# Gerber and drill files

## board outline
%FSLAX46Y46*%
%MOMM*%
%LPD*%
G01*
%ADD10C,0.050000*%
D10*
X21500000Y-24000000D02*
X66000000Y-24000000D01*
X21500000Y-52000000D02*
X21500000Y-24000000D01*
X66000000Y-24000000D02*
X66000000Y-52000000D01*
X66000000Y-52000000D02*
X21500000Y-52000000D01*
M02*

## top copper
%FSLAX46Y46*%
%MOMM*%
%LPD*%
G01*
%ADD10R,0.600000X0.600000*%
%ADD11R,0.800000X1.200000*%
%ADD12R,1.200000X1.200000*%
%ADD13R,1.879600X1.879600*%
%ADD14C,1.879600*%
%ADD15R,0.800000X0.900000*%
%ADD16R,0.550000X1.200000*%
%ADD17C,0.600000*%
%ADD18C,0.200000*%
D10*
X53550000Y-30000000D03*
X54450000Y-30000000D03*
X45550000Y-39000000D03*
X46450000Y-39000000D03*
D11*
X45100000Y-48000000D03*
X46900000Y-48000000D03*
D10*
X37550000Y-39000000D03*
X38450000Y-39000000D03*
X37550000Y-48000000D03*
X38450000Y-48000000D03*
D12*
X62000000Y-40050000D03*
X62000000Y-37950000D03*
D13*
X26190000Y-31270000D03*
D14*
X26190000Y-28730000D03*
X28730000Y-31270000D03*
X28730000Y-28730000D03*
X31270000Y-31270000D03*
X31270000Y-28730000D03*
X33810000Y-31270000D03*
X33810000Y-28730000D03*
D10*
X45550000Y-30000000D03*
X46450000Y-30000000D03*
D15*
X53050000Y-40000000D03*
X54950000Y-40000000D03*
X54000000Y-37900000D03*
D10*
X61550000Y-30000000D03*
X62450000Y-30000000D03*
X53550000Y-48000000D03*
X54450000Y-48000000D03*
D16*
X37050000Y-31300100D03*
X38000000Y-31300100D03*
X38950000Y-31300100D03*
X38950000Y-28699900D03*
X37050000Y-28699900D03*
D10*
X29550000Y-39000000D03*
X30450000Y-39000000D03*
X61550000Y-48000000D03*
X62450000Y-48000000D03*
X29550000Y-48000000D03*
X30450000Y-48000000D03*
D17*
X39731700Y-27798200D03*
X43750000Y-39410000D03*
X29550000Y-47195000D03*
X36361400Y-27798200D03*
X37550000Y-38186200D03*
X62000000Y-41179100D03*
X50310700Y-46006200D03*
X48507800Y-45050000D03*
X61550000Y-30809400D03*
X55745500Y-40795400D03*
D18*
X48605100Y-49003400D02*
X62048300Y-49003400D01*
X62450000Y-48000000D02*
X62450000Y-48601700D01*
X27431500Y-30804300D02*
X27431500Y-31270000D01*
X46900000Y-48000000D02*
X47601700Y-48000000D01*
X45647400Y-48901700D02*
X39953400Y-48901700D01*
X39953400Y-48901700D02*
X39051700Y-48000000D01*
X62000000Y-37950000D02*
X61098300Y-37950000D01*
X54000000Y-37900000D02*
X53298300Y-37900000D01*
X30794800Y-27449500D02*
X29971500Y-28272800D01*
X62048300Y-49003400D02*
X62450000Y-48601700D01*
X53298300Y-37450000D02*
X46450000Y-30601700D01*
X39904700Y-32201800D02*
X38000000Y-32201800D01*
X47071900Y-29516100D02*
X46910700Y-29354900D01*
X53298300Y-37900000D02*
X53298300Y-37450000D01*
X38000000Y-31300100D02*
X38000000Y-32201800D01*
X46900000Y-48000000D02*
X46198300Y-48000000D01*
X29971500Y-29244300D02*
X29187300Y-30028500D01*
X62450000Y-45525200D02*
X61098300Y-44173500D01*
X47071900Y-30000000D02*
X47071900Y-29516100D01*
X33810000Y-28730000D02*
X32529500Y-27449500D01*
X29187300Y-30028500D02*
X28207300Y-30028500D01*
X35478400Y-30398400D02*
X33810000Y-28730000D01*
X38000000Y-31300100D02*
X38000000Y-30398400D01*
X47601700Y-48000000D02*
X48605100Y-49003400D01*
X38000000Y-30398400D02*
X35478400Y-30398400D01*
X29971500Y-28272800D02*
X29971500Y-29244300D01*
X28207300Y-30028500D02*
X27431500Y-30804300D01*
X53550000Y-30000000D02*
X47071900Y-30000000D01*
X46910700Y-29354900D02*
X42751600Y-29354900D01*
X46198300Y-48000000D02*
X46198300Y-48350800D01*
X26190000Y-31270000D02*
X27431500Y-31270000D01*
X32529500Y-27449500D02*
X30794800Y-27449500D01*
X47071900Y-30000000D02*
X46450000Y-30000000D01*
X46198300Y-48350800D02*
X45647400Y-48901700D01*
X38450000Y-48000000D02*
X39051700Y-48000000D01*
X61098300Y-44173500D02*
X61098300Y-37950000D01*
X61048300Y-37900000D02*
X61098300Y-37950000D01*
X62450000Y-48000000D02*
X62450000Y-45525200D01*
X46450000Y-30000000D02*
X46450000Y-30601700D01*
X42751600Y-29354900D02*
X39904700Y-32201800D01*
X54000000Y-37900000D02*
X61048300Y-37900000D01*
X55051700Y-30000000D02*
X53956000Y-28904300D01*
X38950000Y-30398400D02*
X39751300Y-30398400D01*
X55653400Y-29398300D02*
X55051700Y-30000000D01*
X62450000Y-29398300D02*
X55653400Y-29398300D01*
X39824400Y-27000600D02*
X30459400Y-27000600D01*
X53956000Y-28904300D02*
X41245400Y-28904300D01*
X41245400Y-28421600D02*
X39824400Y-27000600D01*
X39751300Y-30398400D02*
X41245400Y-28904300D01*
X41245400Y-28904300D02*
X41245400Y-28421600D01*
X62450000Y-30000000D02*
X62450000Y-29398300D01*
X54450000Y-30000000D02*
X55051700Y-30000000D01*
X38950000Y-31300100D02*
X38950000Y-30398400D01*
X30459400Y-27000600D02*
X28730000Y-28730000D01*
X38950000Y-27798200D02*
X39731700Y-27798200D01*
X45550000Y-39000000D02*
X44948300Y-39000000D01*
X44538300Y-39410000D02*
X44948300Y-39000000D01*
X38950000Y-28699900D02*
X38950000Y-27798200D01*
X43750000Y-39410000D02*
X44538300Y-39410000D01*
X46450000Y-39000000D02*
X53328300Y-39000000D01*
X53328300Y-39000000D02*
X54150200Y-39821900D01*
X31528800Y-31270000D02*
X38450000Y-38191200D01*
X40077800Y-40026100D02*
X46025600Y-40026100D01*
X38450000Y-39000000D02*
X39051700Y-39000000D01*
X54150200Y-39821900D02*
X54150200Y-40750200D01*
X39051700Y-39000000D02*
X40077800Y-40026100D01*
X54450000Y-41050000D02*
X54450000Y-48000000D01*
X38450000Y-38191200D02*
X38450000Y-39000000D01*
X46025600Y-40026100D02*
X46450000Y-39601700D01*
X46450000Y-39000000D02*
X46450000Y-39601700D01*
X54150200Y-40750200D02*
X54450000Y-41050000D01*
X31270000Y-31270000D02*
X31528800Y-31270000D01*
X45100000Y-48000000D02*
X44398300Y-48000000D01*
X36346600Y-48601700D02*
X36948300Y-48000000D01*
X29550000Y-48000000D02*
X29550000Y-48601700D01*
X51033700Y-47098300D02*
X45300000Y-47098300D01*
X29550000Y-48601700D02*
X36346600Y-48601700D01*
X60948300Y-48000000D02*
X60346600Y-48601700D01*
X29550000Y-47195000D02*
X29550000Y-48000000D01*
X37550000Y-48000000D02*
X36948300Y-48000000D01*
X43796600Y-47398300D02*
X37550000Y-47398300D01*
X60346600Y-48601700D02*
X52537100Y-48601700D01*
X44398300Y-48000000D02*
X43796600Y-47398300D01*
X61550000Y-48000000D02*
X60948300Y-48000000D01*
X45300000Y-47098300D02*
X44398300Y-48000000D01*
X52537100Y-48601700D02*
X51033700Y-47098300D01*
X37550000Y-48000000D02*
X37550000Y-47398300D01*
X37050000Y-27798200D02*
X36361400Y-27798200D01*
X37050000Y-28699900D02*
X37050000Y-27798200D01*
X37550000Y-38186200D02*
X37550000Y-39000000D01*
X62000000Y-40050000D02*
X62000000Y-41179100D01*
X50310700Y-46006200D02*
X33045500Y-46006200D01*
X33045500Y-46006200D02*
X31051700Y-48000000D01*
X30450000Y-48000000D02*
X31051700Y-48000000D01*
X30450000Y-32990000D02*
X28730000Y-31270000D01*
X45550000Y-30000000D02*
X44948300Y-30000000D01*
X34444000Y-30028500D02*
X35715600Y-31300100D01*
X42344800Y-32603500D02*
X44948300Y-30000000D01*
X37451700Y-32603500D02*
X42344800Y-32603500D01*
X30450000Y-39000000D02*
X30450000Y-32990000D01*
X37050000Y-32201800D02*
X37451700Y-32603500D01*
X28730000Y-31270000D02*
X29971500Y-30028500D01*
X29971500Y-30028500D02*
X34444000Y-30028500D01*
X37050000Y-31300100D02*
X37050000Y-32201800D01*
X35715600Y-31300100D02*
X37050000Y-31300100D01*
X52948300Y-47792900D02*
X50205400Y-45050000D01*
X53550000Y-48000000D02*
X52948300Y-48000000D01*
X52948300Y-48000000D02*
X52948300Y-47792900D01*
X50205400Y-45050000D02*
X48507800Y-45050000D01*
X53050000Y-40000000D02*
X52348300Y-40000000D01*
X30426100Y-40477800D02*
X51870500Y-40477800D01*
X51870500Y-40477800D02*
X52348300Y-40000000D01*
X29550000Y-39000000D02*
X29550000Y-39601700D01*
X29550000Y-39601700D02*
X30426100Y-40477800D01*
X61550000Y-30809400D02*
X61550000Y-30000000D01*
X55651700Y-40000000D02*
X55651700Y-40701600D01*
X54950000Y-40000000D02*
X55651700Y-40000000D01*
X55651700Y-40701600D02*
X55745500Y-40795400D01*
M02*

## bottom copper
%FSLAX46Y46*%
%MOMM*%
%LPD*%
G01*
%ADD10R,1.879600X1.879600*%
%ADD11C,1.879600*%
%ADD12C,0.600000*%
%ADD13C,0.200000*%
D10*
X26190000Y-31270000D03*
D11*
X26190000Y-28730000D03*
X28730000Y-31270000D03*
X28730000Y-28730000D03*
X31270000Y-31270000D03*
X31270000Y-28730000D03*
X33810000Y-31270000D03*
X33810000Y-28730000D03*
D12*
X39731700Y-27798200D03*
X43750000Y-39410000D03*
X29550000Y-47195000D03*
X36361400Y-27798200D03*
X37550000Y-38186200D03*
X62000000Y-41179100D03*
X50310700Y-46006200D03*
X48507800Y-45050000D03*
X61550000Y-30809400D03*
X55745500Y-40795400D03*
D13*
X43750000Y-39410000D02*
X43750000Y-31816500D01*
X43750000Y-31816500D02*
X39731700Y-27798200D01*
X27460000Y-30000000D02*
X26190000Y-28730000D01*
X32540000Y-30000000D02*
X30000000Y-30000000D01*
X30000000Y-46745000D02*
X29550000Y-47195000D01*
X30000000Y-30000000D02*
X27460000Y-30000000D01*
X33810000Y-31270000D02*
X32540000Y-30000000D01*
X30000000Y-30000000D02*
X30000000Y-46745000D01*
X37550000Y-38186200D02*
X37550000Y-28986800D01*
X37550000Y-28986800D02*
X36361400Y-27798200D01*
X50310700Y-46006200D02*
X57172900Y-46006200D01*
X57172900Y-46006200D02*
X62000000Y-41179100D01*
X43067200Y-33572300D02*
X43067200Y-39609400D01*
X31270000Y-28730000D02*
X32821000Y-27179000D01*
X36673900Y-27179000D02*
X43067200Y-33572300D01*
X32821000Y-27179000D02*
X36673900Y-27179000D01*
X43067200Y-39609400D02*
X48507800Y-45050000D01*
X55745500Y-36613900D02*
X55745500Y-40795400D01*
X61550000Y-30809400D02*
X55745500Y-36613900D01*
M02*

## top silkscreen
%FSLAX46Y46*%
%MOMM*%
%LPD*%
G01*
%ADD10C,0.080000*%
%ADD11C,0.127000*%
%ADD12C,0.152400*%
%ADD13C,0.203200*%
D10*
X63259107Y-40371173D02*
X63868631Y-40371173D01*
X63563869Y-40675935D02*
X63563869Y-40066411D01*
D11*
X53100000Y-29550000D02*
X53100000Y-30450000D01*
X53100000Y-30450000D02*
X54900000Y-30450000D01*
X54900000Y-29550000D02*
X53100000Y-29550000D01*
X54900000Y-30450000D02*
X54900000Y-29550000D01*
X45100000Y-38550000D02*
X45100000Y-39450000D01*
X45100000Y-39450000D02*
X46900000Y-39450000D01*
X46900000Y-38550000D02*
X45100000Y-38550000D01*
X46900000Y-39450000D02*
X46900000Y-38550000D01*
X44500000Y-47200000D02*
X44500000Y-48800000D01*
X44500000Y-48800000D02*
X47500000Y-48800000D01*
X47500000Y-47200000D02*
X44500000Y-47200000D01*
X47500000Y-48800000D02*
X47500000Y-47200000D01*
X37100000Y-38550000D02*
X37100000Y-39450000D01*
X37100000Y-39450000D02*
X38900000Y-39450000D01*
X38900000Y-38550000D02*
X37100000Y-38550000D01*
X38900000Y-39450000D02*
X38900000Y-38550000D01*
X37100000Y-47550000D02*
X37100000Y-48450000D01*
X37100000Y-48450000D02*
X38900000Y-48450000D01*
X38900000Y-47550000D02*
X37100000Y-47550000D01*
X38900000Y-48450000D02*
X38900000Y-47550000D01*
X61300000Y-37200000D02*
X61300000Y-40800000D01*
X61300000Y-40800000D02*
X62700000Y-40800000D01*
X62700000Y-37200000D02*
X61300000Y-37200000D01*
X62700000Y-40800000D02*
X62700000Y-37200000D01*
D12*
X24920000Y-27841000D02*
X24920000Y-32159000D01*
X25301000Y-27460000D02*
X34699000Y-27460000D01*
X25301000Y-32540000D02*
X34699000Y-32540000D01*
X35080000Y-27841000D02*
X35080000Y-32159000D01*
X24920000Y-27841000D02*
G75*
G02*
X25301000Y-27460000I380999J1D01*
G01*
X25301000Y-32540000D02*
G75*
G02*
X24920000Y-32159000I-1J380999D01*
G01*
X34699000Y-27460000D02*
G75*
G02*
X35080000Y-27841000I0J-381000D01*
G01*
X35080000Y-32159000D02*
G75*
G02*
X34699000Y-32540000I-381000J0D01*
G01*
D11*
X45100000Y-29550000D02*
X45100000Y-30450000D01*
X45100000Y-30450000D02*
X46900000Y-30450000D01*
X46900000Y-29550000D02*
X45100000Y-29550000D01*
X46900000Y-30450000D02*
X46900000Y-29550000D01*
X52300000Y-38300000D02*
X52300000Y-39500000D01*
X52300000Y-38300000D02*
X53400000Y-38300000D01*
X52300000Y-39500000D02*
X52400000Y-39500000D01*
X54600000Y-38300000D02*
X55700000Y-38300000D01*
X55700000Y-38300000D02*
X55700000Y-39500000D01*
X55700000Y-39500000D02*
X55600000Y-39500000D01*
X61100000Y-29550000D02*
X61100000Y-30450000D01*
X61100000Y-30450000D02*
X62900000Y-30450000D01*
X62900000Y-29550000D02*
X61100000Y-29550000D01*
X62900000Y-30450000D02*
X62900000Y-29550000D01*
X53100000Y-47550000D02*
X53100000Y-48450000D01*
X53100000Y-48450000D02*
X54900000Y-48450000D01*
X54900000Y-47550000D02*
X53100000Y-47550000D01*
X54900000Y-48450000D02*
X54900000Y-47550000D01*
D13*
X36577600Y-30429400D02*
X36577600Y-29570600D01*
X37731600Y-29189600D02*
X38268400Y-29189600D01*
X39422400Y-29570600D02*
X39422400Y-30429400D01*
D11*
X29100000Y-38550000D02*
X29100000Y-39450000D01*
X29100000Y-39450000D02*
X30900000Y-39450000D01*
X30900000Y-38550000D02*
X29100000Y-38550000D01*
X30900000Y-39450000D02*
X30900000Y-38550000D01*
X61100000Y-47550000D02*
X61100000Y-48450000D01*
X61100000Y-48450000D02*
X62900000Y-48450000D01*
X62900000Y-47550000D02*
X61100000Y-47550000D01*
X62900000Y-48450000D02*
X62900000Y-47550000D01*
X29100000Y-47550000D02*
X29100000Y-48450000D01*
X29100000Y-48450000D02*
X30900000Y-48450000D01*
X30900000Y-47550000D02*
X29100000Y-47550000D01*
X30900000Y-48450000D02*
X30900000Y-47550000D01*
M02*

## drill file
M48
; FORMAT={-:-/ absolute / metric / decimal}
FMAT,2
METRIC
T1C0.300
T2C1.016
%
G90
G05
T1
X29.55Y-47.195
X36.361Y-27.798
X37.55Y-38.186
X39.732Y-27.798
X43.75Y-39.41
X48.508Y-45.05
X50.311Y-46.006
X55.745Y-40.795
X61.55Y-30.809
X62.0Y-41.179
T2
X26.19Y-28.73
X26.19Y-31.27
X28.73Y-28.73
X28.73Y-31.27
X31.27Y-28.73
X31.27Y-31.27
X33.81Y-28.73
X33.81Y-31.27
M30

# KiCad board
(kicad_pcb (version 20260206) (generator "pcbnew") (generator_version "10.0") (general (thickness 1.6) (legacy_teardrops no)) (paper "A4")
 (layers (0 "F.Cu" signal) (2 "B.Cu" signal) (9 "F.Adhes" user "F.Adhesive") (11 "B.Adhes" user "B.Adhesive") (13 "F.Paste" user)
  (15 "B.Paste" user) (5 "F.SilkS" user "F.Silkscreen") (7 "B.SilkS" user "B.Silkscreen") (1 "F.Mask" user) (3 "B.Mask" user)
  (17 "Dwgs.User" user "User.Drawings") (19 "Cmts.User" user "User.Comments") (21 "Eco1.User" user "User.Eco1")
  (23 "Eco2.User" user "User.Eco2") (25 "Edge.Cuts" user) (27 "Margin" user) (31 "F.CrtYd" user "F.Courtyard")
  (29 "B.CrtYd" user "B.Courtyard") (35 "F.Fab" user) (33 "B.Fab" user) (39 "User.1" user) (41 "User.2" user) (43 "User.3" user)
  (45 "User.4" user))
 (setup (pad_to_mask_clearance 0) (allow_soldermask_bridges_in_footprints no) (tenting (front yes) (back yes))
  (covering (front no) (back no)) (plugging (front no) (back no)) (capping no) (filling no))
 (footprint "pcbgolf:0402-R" (layer "F.Cu") (at 54 30)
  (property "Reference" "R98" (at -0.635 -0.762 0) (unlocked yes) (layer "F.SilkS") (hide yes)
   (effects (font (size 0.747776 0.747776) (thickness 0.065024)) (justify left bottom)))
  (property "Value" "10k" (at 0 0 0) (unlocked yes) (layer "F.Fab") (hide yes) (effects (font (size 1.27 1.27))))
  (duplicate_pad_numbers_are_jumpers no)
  (fp_line (start -0.9 -0.45) (end -0.9 0.45) (stroke (width 0.127) (type solid)) (layer "F.SilkS"))
  (fp_line (start -0.9 0.45) (end 0.9 0.45) (stroke (width 0.127) (type solid)) (layer "F.SilkS"))
  (fp_line (start 0.9 -0.45) (end -0.9 -0.45) (stroke (width 0.127) (type solid)) (layer "F.SilkS"))
  (fp_line (start 0.9 0.45) (end 0.9 -0.45) (stroke (width 0.127) (type solid)) (layer "F.SilkS"))
  (pad "1" smd rect (at -0.45 0) (size 0.6 0.6) (layers "F.Cu" "F.Mask" "F.Paste") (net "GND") (solder_mask_margin 0.0508)
   (solder_paste_margin 0) (thermal_bridge_angle 0))
  (pad "2" smd rect (at 0.45 0) (size 0.6 0.6) (layers "F.Cu" "F.Mask" "F.Paste") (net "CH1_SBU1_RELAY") (solder_mask_margin 0.0508)
   (solder_paste_margin 0) (thermal_bridge_angle 0)))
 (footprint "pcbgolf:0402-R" (layer "F.Cu") (at 46 39)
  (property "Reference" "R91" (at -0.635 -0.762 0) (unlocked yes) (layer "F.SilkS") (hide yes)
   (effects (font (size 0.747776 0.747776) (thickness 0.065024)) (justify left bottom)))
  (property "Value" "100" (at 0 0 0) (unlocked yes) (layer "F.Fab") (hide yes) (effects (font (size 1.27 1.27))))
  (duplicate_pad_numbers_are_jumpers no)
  (fp_line (start -0.9 -0.45) (end -0.9 0.45) (stroke (width 0.127) (type solid)) (layer "F.SilkS"))
  (fp_line (start -0.9 0.45) (end 0.9 0.45) (stroke (width 0.127) (type solid)) (layer "F.SilkS"))
  (fp_line (start 0.9 -0.45) (end -0.9 -0.45) (stroke (width 0.127) (type solid)) (layer "F.SilkS"))
  (fp_line (start 0.9 0.45) (end 0.9 -0.45) (stroke (width 0.127) (type solid)) (layer "F.SilkS"))
  (pad "1" smd rect (at -0.45 0) (size 0.6 0.6) (layers "F.Cu" "F.Mask" "F.Paste") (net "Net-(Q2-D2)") (solder_mask_margin 0.0508)
   (solder_paste_margin 0) (thermal_bridge_angle 0))
  (pad "2" smd rect (at 0.45 0) (size 0.6 0.6) (layers "F.Cu" "F.Mask" "F.Paste") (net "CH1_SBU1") (solder_mask_margin 0.0508)
   (solder_paste_margin 0) (thermal_bridge_angle 0)))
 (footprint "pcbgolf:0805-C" (layer "F.Cu") (at 46 48)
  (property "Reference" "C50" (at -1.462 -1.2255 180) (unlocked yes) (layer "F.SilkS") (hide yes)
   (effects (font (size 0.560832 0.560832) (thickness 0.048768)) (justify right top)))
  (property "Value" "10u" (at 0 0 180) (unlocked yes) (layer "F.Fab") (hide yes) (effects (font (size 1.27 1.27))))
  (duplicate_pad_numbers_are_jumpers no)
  (fp_line (start -1.5 -0.8) (end -1.5 0.8) (stroke (width 0.127) (type solid)) (layer "F.SilkS"))
  (fp_line (start -1.5 0.8) (end 1.5 0.8) (stroke (width 0.127) (type solid)) (layer "F.SilkS"))
  (fp_line (start 1.5 -0.8) (end -1.5 -0.8) (stroke (width 0.127) (type solid)) (layer "F.SilkS"))
  (fp_line (start 1.5 0.8) (end 1.5 -0.8) (stroke (width 0.127) (type solid)) (layer "F.SilkS"))
  (pad "1" smd rect (at -0.9 0) (size 0.8 1.2) (layers "F.Cu" "F.Mask" "F.Paste") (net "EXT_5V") (solder_mask_margin 0.0508)
   (solder_paste_margin 0) (thermal_bridge_angle 0))
  (pad "2" smd rect (at 0.9 0) (size 0.8 1.2) (layers "F.Cu" "F.Mask" "F.Paste") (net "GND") (solder_mask_margin 0.0508)
   (solder_paste_margin 0) (thermal_bridge_angle 0)))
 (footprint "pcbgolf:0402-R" (layer "F.Cu") (at 38 39)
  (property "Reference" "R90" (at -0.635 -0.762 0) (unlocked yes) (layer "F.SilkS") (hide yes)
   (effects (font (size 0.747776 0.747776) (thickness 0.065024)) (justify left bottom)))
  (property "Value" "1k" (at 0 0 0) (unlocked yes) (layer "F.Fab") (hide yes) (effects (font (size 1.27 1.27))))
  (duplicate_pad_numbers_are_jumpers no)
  (fp_line (start -0.9 -0.45) (end -0.9 0.45) (stroke (width 0.127) (type solid)) (layer "F.SilkS"))
  (fp_line (start -0.9 0.45) (end 0.9 0.45) (stroke (width 0.127) (type solid)) (layer "F.SilkS"))
  (fp_line (start 0.9 -0.45) (end -0.9 -0.45) (stroke (width 0.127) (type solid)) (layer "F.SilkS"))
  (fp_line (start 0.9 0.45) (end 0.9 -0.45) (stroke (width 0.127) (type solid)) (layer "F.SilkS"))
  (pad "1" smd rect (at -0.45 0) (size 0.6 0.6) (layers "F.Cu" "F.Mask" "F.Paste") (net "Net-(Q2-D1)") (solder_mask_margin 0.0508)
   (solder_paste_margin 0) (thermal_bridge_angle 0))
  (pad "2" smd rect (at 0.45 0) (size 0.6 0.6) (layers "F.Cu" "F.Mask" "F.Paste") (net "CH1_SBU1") (solder_mask_margin 0.0508)
   (solder_paste_margin 0) (thermal_bridge_angle 0)))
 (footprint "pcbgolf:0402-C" (layer "F.Cu") (at 38 48)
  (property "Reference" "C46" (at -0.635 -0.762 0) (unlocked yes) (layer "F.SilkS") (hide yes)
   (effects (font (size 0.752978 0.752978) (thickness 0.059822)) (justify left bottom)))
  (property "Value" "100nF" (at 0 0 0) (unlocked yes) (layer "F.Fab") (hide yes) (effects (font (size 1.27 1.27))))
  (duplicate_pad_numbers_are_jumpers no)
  (fp_line (start -0.9 -0.45) (end -0.9 0.45) (stroke (width 0.127) (type solid)) (layer "F.SilkS"))
  (fp_line (start -0.9 0.45) (end 0.9 0.45) (stroke (width 0.127) (type solid)) (layer "F.SilkS"))
  (fp_line (start 0.9 -0.45) (end -0.9 -0.45) (stroke (width 0.127) (type solid)) (layer "F.SilkS"))
  (fp_line (start 0.9 0.45) (end 0.9 -0.45) (stroke (width 0.127) (type solid)) (layer "F.SilkS"))
  (pad "1" smd rect (at -0.45 0) (size 0.6 0.6) (layers "F.Cu" "F.Mask" "F.Paste") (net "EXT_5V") (solder_mask_margin 0.0508)
   (solder_paste_margin 0) (thermal_bridge_angle 0))
  (pad "2" smd rect (at 0.45 0) (size 0.6 0.6) (layers "F.Cu" "F.Mask" "F.Paste") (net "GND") (solder_mask_margin 0.0508)
   (solder_paste_margin 0) (thermal_bridge_angle 0)))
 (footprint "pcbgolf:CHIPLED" (layer "F.Cu") (at 62 39)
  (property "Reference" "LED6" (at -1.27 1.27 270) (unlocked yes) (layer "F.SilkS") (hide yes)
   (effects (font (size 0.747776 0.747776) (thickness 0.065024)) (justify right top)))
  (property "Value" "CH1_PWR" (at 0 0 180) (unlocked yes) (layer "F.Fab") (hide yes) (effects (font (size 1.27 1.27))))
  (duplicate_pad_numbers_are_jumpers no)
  (fp_line (start -0.7 -1.8) (end -0.7 1.8) (stroke (width 0.127) (type solid)) (layer "F.SilkS"))
  (fp_line (start -0.7 1.8) (end 0.7 1.8) (stroke (width 0.127) (type solid)) (layer "F.SilkS"))
  (fp_line (start 0.7 -1.8) (end -0.7 -1.8) (stroke (width 0.127) (type solid)) (layer "F.SilkS"))
  (fp_line (start 0.7 1.8) (end 0.7 -1.8) (stroke (width 0.127) (type solid)) (layer "F.SilkS"))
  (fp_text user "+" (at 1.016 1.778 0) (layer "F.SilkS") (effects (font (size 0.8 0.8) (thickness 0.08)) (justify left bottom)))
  (pad "A" smd rect (at 0 1.05) (size 1.2 1.2) (layers "F.Cu" "F.Mask" "F.Paste") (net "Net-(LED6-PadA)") (solder_mask_margin 0.0508)
   (solder_paste_margin 0) (thermal_bridge_angle 0))
  (pad "C" smd rect (at 0 -1.05) (size 1.2 1.2) (layers "F.Cu" "F.Mask" "F.Paste") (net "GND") (solder_mask_margin 0.0508)
   (solder_paste_margin 0) (thermal_bridge_angle 0)))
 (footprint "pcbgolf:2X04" (layer "F.Cu") (at 30 30)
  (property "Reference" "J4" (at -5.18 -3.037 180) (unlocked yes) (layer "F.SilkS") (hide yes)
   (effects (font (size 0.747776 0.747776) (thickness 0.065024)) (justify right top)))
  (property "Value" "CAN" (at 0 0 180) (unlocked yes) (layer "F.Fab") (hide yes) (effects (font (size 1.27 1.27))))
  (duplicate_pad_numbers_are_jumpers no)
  (fp_line (start -5.08 -2.159) (end -5.08 2.159) (stroke (width 0.1524) (type solid)) (layer "F.SilkS"))
  (fp_line (start -4.699 -2.54) (end 4.699 -2.54) (stroke (width 0.1524) (type solid)) (layer "F.SilkS"))
  (fp_line (start -4.699 2.54) (end 4.699 2.54) (stroke (width 0.1524) (type solid)) (layer "F.SilkS"))
  (fp_line (start 5.08 -2.159) (end 5.08 2.159) (stroke (width 0.1524) (type solid)) (layer "F.SilkS"))
  (fp_arc (start -5.08 -2.159) (mid -4.968408 -2.428408) (end -4.699 -2.54) (stroke (width 0.1524) (type solid)) (layer "F.SilkS"))
  (fp_arc (start -4.699 2.54) (mid -4.968408 2.428408) (end -5.08 2.159) (stroke (width 0.1524) (type solid)) (layer "F.SilkS"))
  (fp_arc (start 4.699 -2.54) (mid 4.968408 -2.428408) (end 5.08 -2.159) (stroke (width 0.1524) (type solid)) (layer "F.SilkS"))
  (fp_arc (start 5.08 2.159) (mid 4.968408 2.428408) (end 4.699 2.54) (stroke (width 0.1524) (type solid)) (layer "F.SilkS"))
  (pad "1" thru_hole rect (at -3.81 1.27 90) (size 1.8796 1.8796) (drill 1.016) (layers "*.Cu" "*.Mask") (remove_unused_layers no)
   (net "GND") (solder_mask_margin 0.0508) (thermal_bridge_angle 0))
  (pad "2" thru_hole circle (at -3.81 -1.27 90) (size 1.8796 1.8796) (drill 1.016) (layers "*.Cu" "*.Mask") (remove_unused_layers no)
   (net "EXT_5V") (solder_mask_margin 0.0508) (thermal_bridge_angle 0))
  (pad "3" thru_hole circle (at -1.27 1.27 90) (size 1.8796 1.8796) (drill 1.016) (layers "*.Cu" "*.Mask") (remove_unused_layers no)
   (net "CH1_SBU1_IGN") (solder_mask_margin 0.0508) (thermal_bridge_angle 0))
  (pad "4" thru_hole circle (at -1.27 -1.27 90) (size 1.8796 1.8796) (drill 1.016) (layers "*.Cu" "*.Mask") (remove_unused_layers no)
   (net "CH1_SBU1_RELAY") (solder_mask_margin 0.0508) (thermal_bridge_angle 0))
  (pad "5" thru_hole circle (at 1.27 1.27 90) (size 1.8796 1.8796) (drill 1.016) (layers "*.Cu" "*.Mask") (remove_unused_layers no)
   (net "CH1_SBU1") (solder_mask_margin 0.0508) (thermal_bridge_angle 0))
  (pad "6" thru_hole circle (at 1.27 -1.27 90) (size 1.8796 1.8796) (drill 1.016) (layers "*.Cu" "*.Mask") (remove_unused_layers no)
   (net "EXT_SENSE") (solder_mask_margin 0.0508) (thermal_bridge_angle 0))
  (pad "7" thru_hole circle (at 3.81 1.27 90) (size 1.8796 1.8796) (drill 1.016) (layers "*.Cu" "*.Mask") (remove_unused_layers no)
   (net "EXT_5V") (solder_mask_margin 0.0508) (thermal_bridge_angle 0))
  (pad "8" thru_hole circle (at 3.81 -1.27 90) (size 1.8796 1.8796) (drill 1.016) (layers "*.Cu" "*.Mask") (remove_unused_layers no)
   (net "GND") (solder_mask_margin 0.0508) (thermal_bridge_angle 0)))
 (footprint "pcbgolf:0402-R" (layer "F.Cu") (at 46 30)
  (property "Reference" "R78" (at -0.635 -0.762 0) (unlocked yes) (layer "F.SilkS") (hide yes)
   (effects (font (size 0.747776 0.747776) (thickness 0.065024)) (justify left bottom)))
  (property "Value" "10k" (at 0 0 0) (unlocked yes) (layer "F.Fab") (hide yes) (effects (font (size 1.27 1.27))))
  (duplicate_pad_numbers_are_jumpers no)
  (fp_line (start -0.9 -0.45) (end -0.9 0.45) (stroke (width 0.127) (type solid)) (layer "F.SilkS"))
  (fp_line (start -0.9 0.45) (end 0.9 0.45) (stroke (width 0.127) (type solid)) (layer "F.SilkS"))
  (fp_line (start 0.9 -0.45) (end -0.9 -0.45) (stroke (width 0.127) (type solid)) (layer "F.SilkS"))
  (fp_line (start 0.9 0.45) (end 0.9 -0.45) (stroke (width 0.127) (type solid)) (layer "F.SilkS"))
  (pad "1" smd rect (at -0.45 0) (size 0.6 0.6) (layers "F.Cu" "F.Mask" "F.Paste") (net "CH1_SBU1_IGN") (solder_mask_margin 0.0508)
   (solder_paste_margin 0) (thermal_bridge_angle 0))
  (pad "2" smd rect (at 0.45 0) (size 0.6 0.6) (layers "F.Cu" "F.Mask" "F.Paste") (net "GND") (solder_mask_margin 0.0508)
   (solder_paste_margin 0) (thermal_bridge_angle 0)))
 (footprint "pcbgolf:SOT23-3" (layer "F.Cu") (at 54 39)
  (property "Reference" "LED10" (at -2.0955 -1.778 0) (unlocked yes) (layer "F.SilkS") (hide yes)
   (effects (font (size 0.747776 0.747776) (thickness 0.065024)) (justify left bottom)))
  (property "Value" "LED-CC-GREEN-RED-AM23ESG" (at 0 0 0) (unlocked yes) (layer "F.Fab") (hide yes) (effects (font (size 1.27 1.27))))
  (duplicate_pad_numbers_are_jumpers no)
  (fp_line (start -1.7 -0.7) (end -1.7 0.5) (stroke (width 0.127) (type solid)) (layer "F.SilkS"))
  (fp_line (start -1.7 -0.7) (end -0.6 -0.7) (stroke (width 0.127) (type solid)) (layer "F.SilkS"))
  (fp_line (start -1.7 0.5) (end -1.6 0.5) (stroke (width 0.127) (type solid)) (layer "F.SilkS"))
  (fp_line (start 0.6 -0.7) (end 1.7 -0.7) (stroke (width 0.127) (type solid)) (layer "F.SilkS"))
  (fp_line (start 1.7 -0.7) (end 1.7 0.5) (stroke (width 0.127) (type solid)) (layer "F.SilkS"))
  (fp_line (start 1.7 0.5) (end 1.6 0.5) (stroke (width 0.127) (type solid)) (layer "F.SilkS"))
  (pad "1" smd rect (at -0.95 1) (size 0.8 0.9) (layers "F.Cu" "F.Mask" "F.Paste") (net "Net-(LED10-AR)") (solder_mask_margin 0.0508)
   (solder_paste_margin 0) (thermal_bridge_angle 0))
  (pad "2" smd rect (at 0.95 1) (size 0.8 0.9) (layers "F.Cu" "F.Mask" "F.Paste") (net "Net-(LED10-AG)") (solder_mask_margin 0.0508)
   (solder_paste_margin 0) (thermal_bridge_angle 0))
  (pad "3" smd rect (at 0 -1.1) (size 0.8 0.9) (layers "F.Cu" "F.Mask" "F.Paste") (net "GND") (solder_mask_margin 0.0508)
   (solder_paste_margin 0) (thermal_bridge_angle 0)))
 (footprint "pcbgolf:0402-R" (layer "F.Cu") (at 62 30)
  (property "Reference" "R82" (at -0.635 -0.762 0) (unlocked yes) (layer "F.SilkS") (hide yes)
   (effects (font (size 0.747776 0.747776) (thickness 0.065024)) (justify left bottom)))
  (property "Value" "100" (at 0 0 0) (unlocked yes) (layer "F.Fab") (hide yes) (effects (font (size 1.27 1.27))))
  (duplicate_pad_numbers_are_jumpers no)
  (fp_line (start -0.9 -0.45) (end -0.9 0.45) (stroke (width 0.127) (type solid)) (layer "F.SilkS"))
  (fp_line (start -0.9 0.45) (end 0.9 0.45) (stroke (width 0.127) (type solid)) (layer "F.SilkS"))
  (fp_line (start 0.9 -0.45) (end -0.9 -0.45) (stroke (width 0.127) (type solid)) (layer "F.SilkS"))
  (fp_line (start 0.9 0.45) (end 0.9 -0.45) (stroke (width 0.127) (type solid)) (layer "F.SilkS"))
  (pad "1" smd rect (at -0.45 0) (size 0.6 0.6) (layers "F.Cu" "F.Mask" "F.Paste") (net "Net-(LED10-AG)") (solder_mask_margin 0.0508)
   (solder_paste_margin 0) (thermal_bridge_angle 0))
  (pad "2" smd rect (at 0.45 0) (size 0.6 0.6) (layers "F.Cu" "F.Mask" "F.Paste") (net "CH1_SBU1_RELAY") (solder_mask_margin 0.0508)
   (solder_paste_margin 0) (thermal_bridge_angle 0)))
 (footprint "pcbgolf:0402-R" (layer "F.Cu") (at 54 48)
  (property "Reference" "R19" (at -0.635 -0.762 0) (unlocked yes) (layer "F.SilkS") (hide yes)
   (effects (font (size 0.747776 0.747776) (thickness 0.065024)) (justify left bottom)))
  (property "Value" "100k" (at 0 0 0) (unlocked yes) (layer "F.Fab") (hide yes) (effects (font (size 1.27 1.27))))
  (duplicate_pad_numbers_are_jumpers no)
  (fp_line (start -0.9 -0.45) (end -0.9 0.45) (stroke (width 0.127) (type solid)) (layer "F.SilkS"))
  (fp_line (start -0.9 0.45) (end 0.9 0.45) (stroke (width 0.127) (type solid)) (layer "F.SilkS"))
  (fp_line (start 0.9 -0.45) (end -0.9 -0.45) (stroke (width 0.127) (type solid)) (layer "F.SilkS"))
  (fp_line (start 0.9 0.45) (end 0.9 -0.45) (stroke (width 0.127) (type solid)) (layer "F.SilkS"))
  (pad "1" smd rect (at -0.45 0) (size 0.6 0.6) (layers "F.Cu" "F.Mask" "F.Paste") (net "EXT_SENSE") (solder_mask_margin 0.0508)
   (solder_paste_margin 0) (thermal_bridge_angle 0))
  (pad "2" smd rect (at 0.45 0) (size 0.6 0.6) (layers "F.Cu" "F.Mask" "F.Paste") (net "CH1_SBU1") (solder_mask_margin 0.0508)
   (solder_paste_margin 0) (thermal_bridge_angle 0)))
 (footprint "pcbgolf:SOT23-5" (layer "F.Cu") (at 38 30)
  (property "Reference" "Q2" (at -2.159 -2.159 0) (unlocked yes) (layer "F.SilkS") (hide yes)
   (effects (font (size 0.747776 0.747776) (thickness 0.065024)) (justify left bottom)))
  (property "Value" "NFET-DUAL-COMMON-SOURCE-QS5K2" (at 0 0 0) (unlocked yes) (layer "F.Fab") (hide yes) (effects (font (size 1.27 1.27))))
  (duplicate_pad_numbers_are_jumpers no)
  (fp_line (start -1.4224 0.4294) (end -1.4224 -0.4294) (stroke (width 0.2032) (type solid)) (layer "F.SilkS"))
  (fp_line (start -0.2684 -0.8104) (end 0.2684 -0.8104) (stroke (width 0.2032) (type solid)) (layer "F.SilkS"))
  (fp_line (start 1.4224 -0.4294) (end 1.4224 0.4294) (stroke (width 0.2032) (type solid)) (layer "F.SilkS"))
  (pad "1" smd rect (at -0.95 1.3001) (size 0.55 1.2) (layers "F.Cu" "F.Mask" "F.Paste") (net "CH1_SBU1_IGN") (solder_mask_margin 0.0508)
   (solder_paste_margin 0) (thermal_bridge_angle 0))
  (pad "2" smd rect (at 0 1.3001) (size 0.55 1.2) (layers "F.Cu" "F.Mask" "F.Paste") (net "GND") (solder_mask_margin 0.0508)
   (solder_paste_margin 0) (thermal_bridge_angle 0))
  (pad "3" smd rect (at 0.95 1.3001) (size 0.55 1.2) (layers "F.Cu" "F.Mask" "F.Paste") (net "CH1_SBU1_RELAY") (solder_mask_margin 0.0508)
   (solder_paste_margin 0) (thermal_bridge_angle 0))
  (pad "4" smd rect (at 0.95 -1.3001) (size 0.55 1.2) (layers "F.Cu" "F.Mask" "F.Paste") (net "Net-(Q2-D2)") (solder_mask_margin 0.0508)
   (solder_paste_margin 0) (thermal_bridge_angle 0))
  (pad "5" smd rect (at -0.95 -1.3001) (size 0.55 1.2) (layers "F.Cu" "F.Mask" "F.Paste") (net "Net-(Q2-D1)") (solder_mask_margin 0.0508)
   (solder_paste_margin 0) (thermal_bridge_angle 0)))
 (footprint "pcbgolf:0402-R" (layer "F.Cu") (at 30 39)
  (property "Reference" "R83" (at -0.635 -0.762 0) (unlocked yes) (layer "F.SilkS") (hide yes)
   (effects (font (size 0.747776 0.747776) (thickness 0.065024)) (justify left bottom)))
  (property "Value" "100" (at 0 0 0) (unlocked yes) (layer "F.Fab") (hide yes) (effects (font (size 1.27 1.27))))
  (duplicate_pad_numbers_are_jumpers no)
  (fp_line (start -0.9 -0.45) (end -0.9 0.45) (stroke (width 0.127) (type solid)) (layer "F.SilkS"))
  (fp_line (start -0.9 0.45) (end 0.9 0.45) (stroke (width 0.127) (type solid)) (layer "F.SilkS"))
  (fp_line (start 0.9 -0.45) (end -0.9 -0.45) (stroke (width 0.127) (type solid)) (layer "F.SilkS"))
  (fp_line (start 0.9 0.45) (end 0.9 -0.45) (stroke (width 0.127) (type solid)) (layer "F.SilkS"))
  (pad "1" smd rect (at -0.45 0) (size 0.6 0.6) (layers "F.Cu" "F.Mask" "F.Paste") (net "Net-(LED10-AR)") (solder_mask_margin 0.0508)
   (solder_paste_margin 0) (thermal_bridge_angle 0))
  (pad "2" smd rect (at 0.45 0) (size 0.6 0.6) (layers "F.Cu" "F.Mask" "F.Paste") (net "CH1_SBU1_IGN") (solder_mask_margin 0.0508)
   (solder_paste_margin 0) (thermal_bridge_angle 0)))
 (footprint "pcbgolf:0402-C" (layer "F.Cu") (at 62 48)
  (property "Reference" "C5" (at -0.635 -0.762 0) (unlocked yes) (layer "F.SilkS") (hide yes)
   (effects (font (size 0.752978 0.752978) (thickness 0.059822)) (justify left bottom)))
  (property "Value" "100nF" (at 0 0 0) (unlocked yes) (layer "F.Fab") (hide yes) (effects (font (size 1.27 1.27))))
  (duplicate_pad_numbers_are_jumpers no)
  (fp_line (start -0.9 -0.45) (end -0.9 0.45) (stroke (width 0.127) (type solid)) (layer "F.SilkS"))
  (fp_line (start -0.9 0.45) (end 0.9 0.45) (stroke (width 0.127) (type solid)) (layer "F.SilkS"))
  (fp_line (start 0.9 -0.45) (end -0.9 -0.45) (stroke (width 0.127) (type solid)) (layer "F.SilkS"))
  (fp_line (start 0.9 0.45) (end 0.9 -0.45) (stroke (width 0.127) (type solid)) (layer "F.SilkS"))
  (pad "1" smd rect (at -0.45 0) (size 0.6 0.6) (layers "F.Cu" "F.Mask" "F.Paste") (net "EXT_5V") (solder_mask_margin 0.0508)
   (solder_paste_margin 0) (thermal_bridge_angle 0))
  (pad "2" smd rect (at 0.45 0) (size 0.6 0.6) (layers "F.Cu" "F.Mask" "F.Paste") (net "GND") (solder_mask_margin 0.0508)
   (solder_paste_margin 0) (thermal_bridge_angle 0)))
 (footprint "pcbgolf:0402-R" (layer "F.Cu") (at 30 48)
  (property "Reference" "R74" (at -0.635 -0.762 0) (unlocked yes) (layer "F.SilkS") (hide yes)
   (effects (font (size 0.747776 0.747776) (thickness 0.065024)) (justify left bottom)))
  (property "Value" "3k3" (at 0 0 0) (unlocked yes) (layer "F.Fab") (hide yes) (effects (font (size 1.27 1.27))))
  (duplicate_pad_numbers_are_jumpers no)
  (fp_line (start -0.9 -0.45) (end -0.9 0.45) (stroke (width 0.127) (type solid)) (layer "F.SilkS"))
  (fp_line (start -0.9 0.45) (end 0.9 0.45) (stroke (width 0.127) (type solid)) (layer "F.SilkS"))
  (fp_line (start 0.9 -0.45) (end -0.9 -0.45) (stroke (width 0.127) (type solid)) (layer "F.SilkS"))
  (fp_line (start 0.9 0.45) (end 0.9 -0.45) (stroke (width 0.127) (type solid)) (layer "F.SilkS"))
  (pad "1" smd rect (at -0.45 0) (size 0.6 0.6) (layers "F.Cu" "F.Mask" "F.Paste") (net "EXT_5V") (solder_mask_margin 0.0508)
   (solder_paste_margin 0) (thermal_bridge_angle 0))
  (pad "2" smd rect (at 0.45 0) (size 0.6 0.6) (layers "F.Cu" "F.Mask" "F.Paste") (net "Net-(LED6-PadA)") (solder_mask_margin 0.0508)
   (solder_paste_margin 0) (thermal_bridge_angle 0)))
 (gr_line (start 21.5 24) (end 66 24) (stroke (width 0.05) (type default)) (layer "Edge.Cuts"))
 (gr_line (start 21.5 52) (end 21.5 24) (stroke (width 0.05) (type default)) (layer "Edge.Cuts"))
 (gr_line (start 66 24) (end 66 52) (stroke (width 0.05) (type default)) (layer "Edge.Cuts"))
 (gr_line (start 66 52) (end 21.5 52) (stroke (width 0.05) (type default)) (layer "Edge.Cuts"))
 (segment (start 48.6051 49.0034) (end 62.0483 49.0034) (width 0.2) (layer "F.Cu") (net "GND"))
 (segment (start 62.45 48) (end 62.45 48.6017) (width 0.2) (layer "F.Cu") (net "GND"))
 (segment (start 27.4315 30.8043) (end 27.4315 31.27) (width 0.2) (layer "F.Cu") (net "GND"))
 (segment (start 46.9 48) (end 47.6017 48) (width 0.2) (layer "F.Cu") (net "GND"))
 (segment (start 45.6474 48.9017) (end 39.9534 48.9017) (width 0.2) (layer "F.Cu") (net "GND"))
 (segment (start 39.9534 48.9017) (end 39.0517 48) (width 0.2) (layer "F.Cu") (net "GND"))
 (segment (start 62 37.95) (end 61.0983 37.95) (width 0.2) (layer "F.Cu") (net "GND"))
 (segment (start 54 37.9) (end 53.2983 37.9) (width 0.2) (layer "F.Cu") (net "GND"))
 (segment (start 30.7948 27.4495) (end 29.9715 28.2728) (width 0.2) (layer "F.Cu") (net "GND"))
 (segment (start 62.0483 49.0034) (end 62.45 48.6017) (width 0.2) (layer "F.Cu") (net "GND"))
 (segment (start 53.2983 37.45) (end 46.45 30.6017) (width 0.2) (layer "F.Cu") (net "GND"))
 (segment (start 39.9047 32.2018) (end 38 32.2018) (width 0.2) (layer "F.Cu") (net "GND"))
 (segment (start 47.0719 29.5161) (end 46.9107 29.3549) (width 0.2) (layer "F.Cu") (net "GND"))
 (segment (start 53.2983 37.9) (end 53.2983 37.45) (width 0.2) (layer "F.Cu") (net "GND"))
 (segment (start 38 31.3001) (end 38 32.2018) (width 0.2) (layer "F.Cu") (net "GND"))
 (segment (start 46.9 48) (end 46.1983 48) (width 0.2) (layer "F.Cu") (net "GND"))
 (segment (start 29.9715 29.2443) (end 29.1873 30.0285) (width 0.2) (layer "F.Cu") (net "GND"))
 (segment (start 62.45 45.5252) (end 61.0983 44.1735) (width 0.2) (layer "F.Cu") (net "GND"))
 (segment (start 47.0719 30) (end 47.0719 29.5161) (width 0.2) (layer "F.Cu") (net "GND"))
 (segment (start 33.81 28.73) (end 32.5295 27.4495) (width 0.2) (layer "F.Cu") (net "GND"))
 (segment (start 29.1873 30.0285) (end 28.2073 30.0285) (width 0.2) (layer "F.Cu") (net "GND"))
 (segment (start 35.4784 30.3984) (end 33.81 28.73) (width 0.2) (layer "F.Cu") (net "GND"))
 (segment (start 38 31.3001) (end 38 30.3984) (width 0.2) (layer "F.Cu") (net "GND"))
 (segment (start 47.6017 48) (end 48.6051 49.0034) (width 0.2) (layer "F.Cu") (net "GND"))
 (segment (start 38 30.3984) (end 35.4784 30.3984) (width 0.2) (layer "F.Cu") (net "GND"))
 (segment (start 29.9715 28.2728) (end 29.9715 29.2443) (width 0.2) (layer "F.Cu") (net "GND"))
 (segment (start 28.2073 30.0285) (end 27.4315 30.8043) (width 0.2) (layer "F.Cu") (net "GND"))
 (segment (start 53.55 30) (end 47.0719 30) (width 0.2) (layer "F.Cu") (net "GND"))
 (segment (start 46.9107 29.3549) (end 42.7516 29.3549) (width 0.2) (layer "F.Cu") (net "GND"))
 (segment (start 46.1983 48) (end 46.1983 48.3508) (width 0.2) (layer "F.Cu") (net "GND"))
 (segment (start 26.19 31.27) (end 27.4315 31.27) (width 0.2) (layer "F.Cu") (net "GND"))
 (segment (start 32.5295 27.4495) (end 30.7948 27.4495) (width 0.2) (layer "F.Cu") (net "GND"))
 (segment (start 47.0719 30) (end 46.45 30) (width 0.2) (layer "F.Cu") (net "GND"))
 (segment (start 46.1983 48.3508) (end 45.6474 48.9017) (width 0.2) (layer "F.Cu") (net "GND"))
 (segment (start 38.45 48) (end 39.0517 48) (width 0.2) (layer "F.Cu") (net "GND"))
 (segment (start 61.0983 44.1735) (end 61.0983 37.95) (width 0.2) (layer "F.Cu") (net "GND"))
 (segment (start 61.0483 37.9) (end 61.0983 37.95) (width 0.2) (layer "F.Cu") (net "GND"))
 (segment (start 62.45 48) (end 62.45 45.5252) (width 0.2) (layer "F.Cu") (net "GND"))
 (segment (start 46.45 30) (end 46.45 30.6017) (width 0.2) (layer "F.Cu") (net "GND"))
 (segment (start 42.7516 29.3549) (end 39.9047 32.2018) (width 0.2) (layer "F.Cu") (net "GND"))
 (segment (start 54 37.9) (end 61.0483 37.9) (width 0.2) (layer "F.Cu") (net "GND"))
 (segment (start 55.0517 30) (end 53.956 28.9043) (width 0.2) (layer "F.Cu") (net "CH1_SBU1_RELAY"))
 (segment (start 38.95 30.3984) (end 39.7513 30.3984) (width 0.2) (layer "F.Cu") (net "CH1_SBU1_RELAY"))
 (segment (start 55.6534 29.3983) (end 55.0517 30) (width 0.2) (layer "F.Cu") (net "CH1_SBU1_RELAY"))
 (segment (start 62.45 29.3983) (end 55.6534 29.3983) (width 0.2) (layer "F.Cu") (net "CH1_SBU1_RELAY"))
 (segment (start 39.8244 27.0006) (end 30.4594 27.0006) (width 0.2) (layer "F.Cu") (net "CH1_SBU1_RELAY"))
 (segment (start 53.956 28.9043) (end 41.2454 28.9043) (width 0.2) (layer "F.Cu") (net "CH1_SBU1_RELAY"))
 (segment (start 41.2454 28.4216) (end 39.8244 27.0006) (width 0.2) (layer "F.Cu") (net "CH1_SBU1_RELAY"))
 (segment (start 39.7513 30.3984) (end 41.2454 28.9043) (width 0.2) (layer "F.Cu") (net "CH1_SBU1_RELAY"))
 (segment (start 41.2454 28.9043) (end 41.2454 28.4216) (width 0.2) (layer "F.Cu") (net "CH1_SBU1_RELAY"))
 (segment (start 62.45 30) (end 62.45 29.3983) (width 0.2) (layer "F.Cu") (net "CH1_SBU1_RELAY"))
 (segment (start 54.45 30) (end 55.0517 30) (width 0.2) (layer "F.Cu") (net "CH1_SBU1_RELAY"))
 (segment (start 38.95 31.3001) (end 38.95 30.3984) (width 0.2) (layer "F.Cu") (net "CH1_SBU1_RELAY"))
 (segment (start 30.4594 27.0006) (end 28.73 28.73) (width 0.2) (layer "F.Cu") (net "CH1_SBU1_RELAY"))
 (segment (start 38.95 27.7982) (end 39.7317 27.7982) (width 0.2) (layer "F.Cu") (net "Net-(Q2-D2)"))
 (segment (start 45.55 39) (end 44.9483 39) (width 0.2) (layer "F.Cu") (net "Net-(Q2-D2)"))
 (segment (start 44.5383 39.41) (end 44.9483 39) (width 0.2) (layer "F.Cu") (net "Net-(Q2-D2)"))
 (segment (start 38.95 28.6999) (end 38.95 27.7982) (width 0.2) (layer "F.Cu") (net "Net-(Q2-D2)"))
 (segment (start 43.75 39.41) (end 44.5383 39.41) (width 0.2) (layer "F.Cu") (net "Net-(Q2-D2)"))
 (via (at 39.7317 27.7982) (size 0.6) (drill 0.3) (layers "F.Cu" "B.Cu") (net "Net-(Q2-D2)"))
 (via (at 43.75 39.41) (size 0.6) (drill 0.3) (layers "F.Cu" "B.Cu") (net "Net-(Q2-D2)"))
 (segment (start 43.75 39.41) (end 43.75 31.8165) (width 0.2) (layer "B.Cu") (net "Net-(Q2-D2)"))
 (segment (start 43.75 31.8165) (end 39.7317 27.7982) (width 0.2) (layer "B.Cu") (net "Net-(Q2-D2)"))
 (segment (start 46.45 39) (end 53.3283 39) (width 0.2) (layer "F.Cu") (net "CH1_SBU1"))
 (segment (start 53.3283 39) (end 54.1502 39.8219) (width 0.2) (layer "F.Cu") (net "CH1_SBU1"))
 (segment (start 31.5288 31.27) (end 38.45 38.1912) (width 0.2) (layer "F.Cu") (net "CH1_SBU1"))
 (segment (start 40.0778 40.0261) (end 46.0256 40.0261) (width 0.2) (layer "F.Cu") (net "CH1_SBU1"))
 (segment (start 38.45 39) (end 39.0517 39) (width 0.2) (layer "F.Cu") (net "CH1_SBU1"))
 (segment (start 54.1502 39.8219) (end 54.1502 40.7502) (width 0.2) (layer "F.Cu") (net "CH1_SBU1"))
 (segment (start 39.0517 39) (end 40.0778 40.0261) (width 0.2) (layer "F.Cu") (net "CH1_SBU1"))
 (segment (start 54.45 41.05) (end 54.45 48) (width 0.2) (layer "F.Cu") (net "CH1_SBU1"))
 (segment (start 38.45 38.1912) (end 38.45 39) (width 0.2) (layer "F.Cu") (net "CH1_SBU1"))
 (segment (start 46.0256 40.0261) (end 46.45 39.6017) (width 0.2) (layer "F.Cu") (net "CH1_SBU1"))
 (segment (start 46.45 39) (end 46.45 39.6017) (width 0.2) (layer "F.Cu") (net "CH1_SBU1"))
 (segment (start 54.1502 40.7502) (end 54.45 41.05) (width 0.2) (layer "F.Cu") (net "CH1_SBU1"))
 (segment (start 31.27 31.27) (end 31.5288 31.27) (width 0.2) (layer "F.Cu") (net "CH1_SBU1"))
 (segment (start 45.1 48) (end 44.3983 48) (width 0.2) (layer "F.Cu") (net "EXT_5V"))
 (segment (start 36.3466 48.6017) (end 36.9483 48) (width 0.2) (layer "F.Cu") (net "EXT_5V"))
 (segment (start 29.55 48) (end 29.55 48.6017) (width 0.2) (layer "F.Cu") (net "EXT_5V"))
 (segment (start 51.0337 47.0983) (end 45.3 47.0983) (width 0.2) (layer "F.Cu") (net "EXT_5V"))
 (segment (start 29.55 48.6017) (end 36.3466 48.6017) (width 0.2) (layer "F.Cu") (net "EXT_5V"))
 (segment (start 60.9483 48) (end 60.3466 48.6017) (width 0.2) (layer "F.Cu") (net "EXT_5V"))
 (segment (start 29.55 47.195) (end 29.55 48) (width 0.2) (layer "F.Cu") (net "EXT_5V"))
 (segment (start 37.55 48) (end 36.9483 48) (width 0.2) (layer "F.Cu") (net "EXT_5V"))
 (segment (start 43.7966 47.3983) (end 37.55 47.3983) (width 0.2) (layer "F.Cu") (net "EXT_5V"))
 (segment (start 60.3466 48.6017) (end 52.5371 48.6017) (width 0.2) (layer "F.Cu") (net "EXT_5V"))
 (segment (start 44.3983 48) (end 43.7966 47.3983) (width 0.2) (layer "F.Cu") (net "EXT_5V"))
 (segment (start 61.55 48) (end 60.9483 48) (width 0.2) (layer "F.Cu") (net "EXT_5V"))
 (segment (start 45.3 47.0983) (end 44.3983 48) (width 0.2) (layer "F.Cu") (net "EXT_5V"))
 (segment (start 52.5371 48.6017) (end 51.0337 47.0983) (width 0.2) (layer "F.Cu") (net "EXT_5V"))
 (segment (start 37.55 48) (end 37.55 47.3983) (width 0.2) (layer "F.Cu") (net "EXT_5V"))
 (via (at 29.55 47.195) (size 0.6) (drill 0.3) (layers "F.Cu" "B.Cu") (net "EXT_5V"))
 (segment (start 27.46 30) (end 26.19 28.73) (width 0.2) (layer "B.Cu") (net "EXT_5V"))
 (segment (start 32.54 30) (end 30 30) (width 0.2) (layer "B.Cu") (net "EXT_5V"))
 (segment (start 30 46.745) (end 29.55 47.195) (width 0.2) (layer "B.Cu") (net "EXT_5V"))
 (segment (start 30 30) (end 27.46 30) (width 0.2) (layer "B.Cu") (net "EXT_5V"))
 (segment (start 33.81 31.27) (end 32.54 30) (width 0.2) (layer "B.Cu") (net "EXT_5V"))
 (segment (start 30 30) (end 30 46.745) (width 0.2) (layer "B.Cu") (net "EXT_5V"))
 (segment (start 37.05 27.7982) (end 36.3614 27.7982) (width 0.2) (layer "F.Cu") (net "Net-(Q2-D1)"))
 (segment (start 37.05 28.6999) (end 37.05 27.7982) (width 0.2) (layer "F.Cu") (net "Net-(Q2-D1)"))
 (segment (start 37.55 38.1862) (end 37.55 39) (width 0.2) (layer "F.Cu") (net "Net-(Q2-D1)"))
 (via (at 36.3614 27.7982) (size 0.6) (drill 0.3) (layers "F.Cu" "B.Cu") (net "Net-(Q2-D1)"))
 (via (at 37.55 38.1862) (size 0.6) (drill 0.3) (layers "F.Cu" "B.Cu") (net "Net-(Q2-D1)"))
 (segment (start 37.55 38.1862) (end 37.55 28.9868) (width 0.2) (layer "B.Cu") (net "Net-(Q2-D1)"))
 (segment (start 37.55 28.9868) (end 36.3614 27.7982) (width 0.2) (layer "B.Cu") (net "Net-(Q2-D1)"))
 (segment (start 62 40.05) (end 62 41.1791) (width 0.2) (layer "F.Cu") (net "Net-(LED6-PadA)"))
 (segment (start 50.3107 46.0062) (end 33.0455 46.0062) (width 0.2) (layer "F.Cu") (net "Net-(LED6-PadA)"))
 (segment (start 33.0455 46.0062) (end 31.0517 48) (width 0.2) (layer "F.Cu") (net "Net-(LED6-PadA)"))
 (segment (start 30.45 48) (end 31.0517 48) (width 0.2) (layer "F.Cu") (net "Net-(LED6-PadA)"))
 (via (at 62 41.1791) (size 0.6) (drill 0.3) (layers "F.Cu" "B.Cu") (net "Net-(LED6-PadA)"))
 (via (at 50.3107 46.0062) (size 0.6) (drill 0.3) (layers "F.Cu" "B.Cu") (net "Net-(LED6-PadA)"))
 (segment (start 50.3107 46.0062) (end 57.1729 46.0062) (width 0.2) (layer "B.Cu") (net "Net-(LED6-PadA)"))
 (segment (start 57.1729 46.0062) (end 62 41.1791) (width 0.2) (layer "B.Cu") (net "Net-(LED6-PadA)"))
 (segment (start 30.45 32.99) (end 28.73 31.27) (width 0.2) (layer "F.Cu") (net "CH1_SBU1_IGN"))
 (segment (start 45.55 30) (end 44.9483 30) (width 0.2) (layer "F.Cu") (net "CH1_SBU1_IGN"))
 (segment (start 34.444 30.0285) (end 35.7156 31.3001) (width 0.2) (layer "F.Cu") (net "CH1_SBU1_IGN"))
 (segment (start 42.3448 32.6035) (end 44.9483 30) (width 0.2) (layer "F.Cu") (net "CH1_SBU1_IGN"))
 (segment (start 37.4517 32.6035) (end 42.3448 32.6035) (width 0.2) (layer "F.Cu") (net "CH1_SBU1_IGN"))
 (segment (start 30.45 39) (end 30.45 32.99) (width 0.2) (layer "F.Cu") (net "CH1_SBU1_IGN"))
 (segment (start 37.05 32.2018) (end 37.4517 32.6035) (width 0.2) (layer "F.Cu") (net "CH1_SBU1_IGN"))
 (segment (start 28.73 31.27) (end 29.9715 30.0285) (width 0.2) (layer "F.Cu") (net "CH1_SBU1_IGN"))
 (segment (start 29.9715 30.0285) (end 34.444 30.0285) (width 0.2) (layer "F.Cu") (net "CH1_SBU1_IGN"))
 (segment (start 37.05 31.3001) (end 37.05 32.2018) (width 0.2) (layer "F.Cu") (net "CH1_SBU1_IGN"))
 (segment (start 35.7156 31.3001) (end 37.05 31.3001) (width 0.2) (layer "F.Cu") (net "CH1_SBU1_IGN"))
 (segment (start 52.9483 47.7929) (end 50.2054 45.05) (width 0.2) (layer "F.Cu") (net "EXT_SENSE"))
 (segment (start 53.55 48) (end 52.9483 48) (width 0.2) (layer "F.Cu") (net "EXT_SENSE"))
 (segment (start 52.9483 48) (end 52.9483 47.7929) (width 0.2) (layer "F.Cu") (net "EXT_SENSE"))
 (segment (start 50.2054 45.05) (end 48.5078 45.05) (width 0.2) (layer "F.Cu") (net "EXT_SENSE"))
 (via (at 48.5078 45.05) (size 0.6) (drill 0.3) (layers "F.Cu" "B.Cu") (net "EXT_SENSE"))
 (segment (start 43.0672 33.5723) (end 43.0672 39.6094) (width 0.2) (layer "B.Cu") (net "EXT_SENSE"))
 (segment (start 31.27 28.73) (end 32.821 27.179) (width 0.2) (layer "B.Cu") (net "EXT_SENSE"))
 (segment (start 36.6739 27.179) (end 43.0672 33.5723) (width 0.2) (layer "B.Cu") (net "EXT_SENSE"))
 (segment (start 32.821 27.179) (end 36.6739 27.179) (width 0.2) (layer "B.Cu") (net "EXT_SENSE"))
 (segment (start 43.0672 39.6094) (end 48.5078 45.05) (width 0.2) (layer "B.Cu") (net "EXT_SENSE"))
 (segment (start 53.05 40) (end 52.3483 40) (width 0.2) (layer "F.Cu") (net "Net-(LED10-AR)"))
 (segment (start 30.4261 40.4778) (end 51.8705 40.4778) (width 0.2) (layer "F.Cu") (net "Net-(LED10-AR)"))
 (segment (start 51.8705 40.4778) (end 52.3483 40) (width 0.2) (layer "F.Cu") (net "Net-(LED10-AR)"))
 (segment (start 29.55 39) (end 29.55 39.6017) (width 0.2) (layer "F.Cu") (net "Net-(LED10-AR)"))
 (segment (start 29.55 39.6017) (end 30.4261 40.4778) (width 0.2) (layer "F.Cu") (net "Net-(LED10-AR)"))
 (segment (start 61.55 30.8094) (end 61.55 30) (width 0.2) (layer "F.Cu") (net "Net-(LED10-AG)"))
 (segment (start 55.6517 40) (end 55.6517 40.7016) (width 0.2) (layer "F.Cu") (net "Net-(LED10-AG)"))
 (segment (start 54.95 40) (end 55.6517 40) (width 0.2) (layer "F.Cu") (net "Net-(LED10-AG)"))
 (segment (start 55.6517 40.7016) (end 55.7455 40.7954) (width 0.2) (layer "F.Cu") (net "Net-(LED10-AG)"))
 (via (at 61.55 30.8094) (size 0.6) (drill 0.3) (layers "F.Cu" "B.Cu") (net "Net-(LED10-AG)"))
 (via (at 55.7455 40.7954) (size 0.6) (drill 0.3) (layers "F.Cu" "B.Cu") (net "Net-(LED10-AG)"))
 (segment (start 55.7455 36.6139) (end 55.7455 40.7954) (width 0.2) (layer "B.Cu") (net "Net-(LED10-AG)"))
 (segment (start 61.55 30.8094) (end 55.7455 36.6139) (width 0.2) (layer "B.Cu") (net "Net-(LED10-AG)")))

